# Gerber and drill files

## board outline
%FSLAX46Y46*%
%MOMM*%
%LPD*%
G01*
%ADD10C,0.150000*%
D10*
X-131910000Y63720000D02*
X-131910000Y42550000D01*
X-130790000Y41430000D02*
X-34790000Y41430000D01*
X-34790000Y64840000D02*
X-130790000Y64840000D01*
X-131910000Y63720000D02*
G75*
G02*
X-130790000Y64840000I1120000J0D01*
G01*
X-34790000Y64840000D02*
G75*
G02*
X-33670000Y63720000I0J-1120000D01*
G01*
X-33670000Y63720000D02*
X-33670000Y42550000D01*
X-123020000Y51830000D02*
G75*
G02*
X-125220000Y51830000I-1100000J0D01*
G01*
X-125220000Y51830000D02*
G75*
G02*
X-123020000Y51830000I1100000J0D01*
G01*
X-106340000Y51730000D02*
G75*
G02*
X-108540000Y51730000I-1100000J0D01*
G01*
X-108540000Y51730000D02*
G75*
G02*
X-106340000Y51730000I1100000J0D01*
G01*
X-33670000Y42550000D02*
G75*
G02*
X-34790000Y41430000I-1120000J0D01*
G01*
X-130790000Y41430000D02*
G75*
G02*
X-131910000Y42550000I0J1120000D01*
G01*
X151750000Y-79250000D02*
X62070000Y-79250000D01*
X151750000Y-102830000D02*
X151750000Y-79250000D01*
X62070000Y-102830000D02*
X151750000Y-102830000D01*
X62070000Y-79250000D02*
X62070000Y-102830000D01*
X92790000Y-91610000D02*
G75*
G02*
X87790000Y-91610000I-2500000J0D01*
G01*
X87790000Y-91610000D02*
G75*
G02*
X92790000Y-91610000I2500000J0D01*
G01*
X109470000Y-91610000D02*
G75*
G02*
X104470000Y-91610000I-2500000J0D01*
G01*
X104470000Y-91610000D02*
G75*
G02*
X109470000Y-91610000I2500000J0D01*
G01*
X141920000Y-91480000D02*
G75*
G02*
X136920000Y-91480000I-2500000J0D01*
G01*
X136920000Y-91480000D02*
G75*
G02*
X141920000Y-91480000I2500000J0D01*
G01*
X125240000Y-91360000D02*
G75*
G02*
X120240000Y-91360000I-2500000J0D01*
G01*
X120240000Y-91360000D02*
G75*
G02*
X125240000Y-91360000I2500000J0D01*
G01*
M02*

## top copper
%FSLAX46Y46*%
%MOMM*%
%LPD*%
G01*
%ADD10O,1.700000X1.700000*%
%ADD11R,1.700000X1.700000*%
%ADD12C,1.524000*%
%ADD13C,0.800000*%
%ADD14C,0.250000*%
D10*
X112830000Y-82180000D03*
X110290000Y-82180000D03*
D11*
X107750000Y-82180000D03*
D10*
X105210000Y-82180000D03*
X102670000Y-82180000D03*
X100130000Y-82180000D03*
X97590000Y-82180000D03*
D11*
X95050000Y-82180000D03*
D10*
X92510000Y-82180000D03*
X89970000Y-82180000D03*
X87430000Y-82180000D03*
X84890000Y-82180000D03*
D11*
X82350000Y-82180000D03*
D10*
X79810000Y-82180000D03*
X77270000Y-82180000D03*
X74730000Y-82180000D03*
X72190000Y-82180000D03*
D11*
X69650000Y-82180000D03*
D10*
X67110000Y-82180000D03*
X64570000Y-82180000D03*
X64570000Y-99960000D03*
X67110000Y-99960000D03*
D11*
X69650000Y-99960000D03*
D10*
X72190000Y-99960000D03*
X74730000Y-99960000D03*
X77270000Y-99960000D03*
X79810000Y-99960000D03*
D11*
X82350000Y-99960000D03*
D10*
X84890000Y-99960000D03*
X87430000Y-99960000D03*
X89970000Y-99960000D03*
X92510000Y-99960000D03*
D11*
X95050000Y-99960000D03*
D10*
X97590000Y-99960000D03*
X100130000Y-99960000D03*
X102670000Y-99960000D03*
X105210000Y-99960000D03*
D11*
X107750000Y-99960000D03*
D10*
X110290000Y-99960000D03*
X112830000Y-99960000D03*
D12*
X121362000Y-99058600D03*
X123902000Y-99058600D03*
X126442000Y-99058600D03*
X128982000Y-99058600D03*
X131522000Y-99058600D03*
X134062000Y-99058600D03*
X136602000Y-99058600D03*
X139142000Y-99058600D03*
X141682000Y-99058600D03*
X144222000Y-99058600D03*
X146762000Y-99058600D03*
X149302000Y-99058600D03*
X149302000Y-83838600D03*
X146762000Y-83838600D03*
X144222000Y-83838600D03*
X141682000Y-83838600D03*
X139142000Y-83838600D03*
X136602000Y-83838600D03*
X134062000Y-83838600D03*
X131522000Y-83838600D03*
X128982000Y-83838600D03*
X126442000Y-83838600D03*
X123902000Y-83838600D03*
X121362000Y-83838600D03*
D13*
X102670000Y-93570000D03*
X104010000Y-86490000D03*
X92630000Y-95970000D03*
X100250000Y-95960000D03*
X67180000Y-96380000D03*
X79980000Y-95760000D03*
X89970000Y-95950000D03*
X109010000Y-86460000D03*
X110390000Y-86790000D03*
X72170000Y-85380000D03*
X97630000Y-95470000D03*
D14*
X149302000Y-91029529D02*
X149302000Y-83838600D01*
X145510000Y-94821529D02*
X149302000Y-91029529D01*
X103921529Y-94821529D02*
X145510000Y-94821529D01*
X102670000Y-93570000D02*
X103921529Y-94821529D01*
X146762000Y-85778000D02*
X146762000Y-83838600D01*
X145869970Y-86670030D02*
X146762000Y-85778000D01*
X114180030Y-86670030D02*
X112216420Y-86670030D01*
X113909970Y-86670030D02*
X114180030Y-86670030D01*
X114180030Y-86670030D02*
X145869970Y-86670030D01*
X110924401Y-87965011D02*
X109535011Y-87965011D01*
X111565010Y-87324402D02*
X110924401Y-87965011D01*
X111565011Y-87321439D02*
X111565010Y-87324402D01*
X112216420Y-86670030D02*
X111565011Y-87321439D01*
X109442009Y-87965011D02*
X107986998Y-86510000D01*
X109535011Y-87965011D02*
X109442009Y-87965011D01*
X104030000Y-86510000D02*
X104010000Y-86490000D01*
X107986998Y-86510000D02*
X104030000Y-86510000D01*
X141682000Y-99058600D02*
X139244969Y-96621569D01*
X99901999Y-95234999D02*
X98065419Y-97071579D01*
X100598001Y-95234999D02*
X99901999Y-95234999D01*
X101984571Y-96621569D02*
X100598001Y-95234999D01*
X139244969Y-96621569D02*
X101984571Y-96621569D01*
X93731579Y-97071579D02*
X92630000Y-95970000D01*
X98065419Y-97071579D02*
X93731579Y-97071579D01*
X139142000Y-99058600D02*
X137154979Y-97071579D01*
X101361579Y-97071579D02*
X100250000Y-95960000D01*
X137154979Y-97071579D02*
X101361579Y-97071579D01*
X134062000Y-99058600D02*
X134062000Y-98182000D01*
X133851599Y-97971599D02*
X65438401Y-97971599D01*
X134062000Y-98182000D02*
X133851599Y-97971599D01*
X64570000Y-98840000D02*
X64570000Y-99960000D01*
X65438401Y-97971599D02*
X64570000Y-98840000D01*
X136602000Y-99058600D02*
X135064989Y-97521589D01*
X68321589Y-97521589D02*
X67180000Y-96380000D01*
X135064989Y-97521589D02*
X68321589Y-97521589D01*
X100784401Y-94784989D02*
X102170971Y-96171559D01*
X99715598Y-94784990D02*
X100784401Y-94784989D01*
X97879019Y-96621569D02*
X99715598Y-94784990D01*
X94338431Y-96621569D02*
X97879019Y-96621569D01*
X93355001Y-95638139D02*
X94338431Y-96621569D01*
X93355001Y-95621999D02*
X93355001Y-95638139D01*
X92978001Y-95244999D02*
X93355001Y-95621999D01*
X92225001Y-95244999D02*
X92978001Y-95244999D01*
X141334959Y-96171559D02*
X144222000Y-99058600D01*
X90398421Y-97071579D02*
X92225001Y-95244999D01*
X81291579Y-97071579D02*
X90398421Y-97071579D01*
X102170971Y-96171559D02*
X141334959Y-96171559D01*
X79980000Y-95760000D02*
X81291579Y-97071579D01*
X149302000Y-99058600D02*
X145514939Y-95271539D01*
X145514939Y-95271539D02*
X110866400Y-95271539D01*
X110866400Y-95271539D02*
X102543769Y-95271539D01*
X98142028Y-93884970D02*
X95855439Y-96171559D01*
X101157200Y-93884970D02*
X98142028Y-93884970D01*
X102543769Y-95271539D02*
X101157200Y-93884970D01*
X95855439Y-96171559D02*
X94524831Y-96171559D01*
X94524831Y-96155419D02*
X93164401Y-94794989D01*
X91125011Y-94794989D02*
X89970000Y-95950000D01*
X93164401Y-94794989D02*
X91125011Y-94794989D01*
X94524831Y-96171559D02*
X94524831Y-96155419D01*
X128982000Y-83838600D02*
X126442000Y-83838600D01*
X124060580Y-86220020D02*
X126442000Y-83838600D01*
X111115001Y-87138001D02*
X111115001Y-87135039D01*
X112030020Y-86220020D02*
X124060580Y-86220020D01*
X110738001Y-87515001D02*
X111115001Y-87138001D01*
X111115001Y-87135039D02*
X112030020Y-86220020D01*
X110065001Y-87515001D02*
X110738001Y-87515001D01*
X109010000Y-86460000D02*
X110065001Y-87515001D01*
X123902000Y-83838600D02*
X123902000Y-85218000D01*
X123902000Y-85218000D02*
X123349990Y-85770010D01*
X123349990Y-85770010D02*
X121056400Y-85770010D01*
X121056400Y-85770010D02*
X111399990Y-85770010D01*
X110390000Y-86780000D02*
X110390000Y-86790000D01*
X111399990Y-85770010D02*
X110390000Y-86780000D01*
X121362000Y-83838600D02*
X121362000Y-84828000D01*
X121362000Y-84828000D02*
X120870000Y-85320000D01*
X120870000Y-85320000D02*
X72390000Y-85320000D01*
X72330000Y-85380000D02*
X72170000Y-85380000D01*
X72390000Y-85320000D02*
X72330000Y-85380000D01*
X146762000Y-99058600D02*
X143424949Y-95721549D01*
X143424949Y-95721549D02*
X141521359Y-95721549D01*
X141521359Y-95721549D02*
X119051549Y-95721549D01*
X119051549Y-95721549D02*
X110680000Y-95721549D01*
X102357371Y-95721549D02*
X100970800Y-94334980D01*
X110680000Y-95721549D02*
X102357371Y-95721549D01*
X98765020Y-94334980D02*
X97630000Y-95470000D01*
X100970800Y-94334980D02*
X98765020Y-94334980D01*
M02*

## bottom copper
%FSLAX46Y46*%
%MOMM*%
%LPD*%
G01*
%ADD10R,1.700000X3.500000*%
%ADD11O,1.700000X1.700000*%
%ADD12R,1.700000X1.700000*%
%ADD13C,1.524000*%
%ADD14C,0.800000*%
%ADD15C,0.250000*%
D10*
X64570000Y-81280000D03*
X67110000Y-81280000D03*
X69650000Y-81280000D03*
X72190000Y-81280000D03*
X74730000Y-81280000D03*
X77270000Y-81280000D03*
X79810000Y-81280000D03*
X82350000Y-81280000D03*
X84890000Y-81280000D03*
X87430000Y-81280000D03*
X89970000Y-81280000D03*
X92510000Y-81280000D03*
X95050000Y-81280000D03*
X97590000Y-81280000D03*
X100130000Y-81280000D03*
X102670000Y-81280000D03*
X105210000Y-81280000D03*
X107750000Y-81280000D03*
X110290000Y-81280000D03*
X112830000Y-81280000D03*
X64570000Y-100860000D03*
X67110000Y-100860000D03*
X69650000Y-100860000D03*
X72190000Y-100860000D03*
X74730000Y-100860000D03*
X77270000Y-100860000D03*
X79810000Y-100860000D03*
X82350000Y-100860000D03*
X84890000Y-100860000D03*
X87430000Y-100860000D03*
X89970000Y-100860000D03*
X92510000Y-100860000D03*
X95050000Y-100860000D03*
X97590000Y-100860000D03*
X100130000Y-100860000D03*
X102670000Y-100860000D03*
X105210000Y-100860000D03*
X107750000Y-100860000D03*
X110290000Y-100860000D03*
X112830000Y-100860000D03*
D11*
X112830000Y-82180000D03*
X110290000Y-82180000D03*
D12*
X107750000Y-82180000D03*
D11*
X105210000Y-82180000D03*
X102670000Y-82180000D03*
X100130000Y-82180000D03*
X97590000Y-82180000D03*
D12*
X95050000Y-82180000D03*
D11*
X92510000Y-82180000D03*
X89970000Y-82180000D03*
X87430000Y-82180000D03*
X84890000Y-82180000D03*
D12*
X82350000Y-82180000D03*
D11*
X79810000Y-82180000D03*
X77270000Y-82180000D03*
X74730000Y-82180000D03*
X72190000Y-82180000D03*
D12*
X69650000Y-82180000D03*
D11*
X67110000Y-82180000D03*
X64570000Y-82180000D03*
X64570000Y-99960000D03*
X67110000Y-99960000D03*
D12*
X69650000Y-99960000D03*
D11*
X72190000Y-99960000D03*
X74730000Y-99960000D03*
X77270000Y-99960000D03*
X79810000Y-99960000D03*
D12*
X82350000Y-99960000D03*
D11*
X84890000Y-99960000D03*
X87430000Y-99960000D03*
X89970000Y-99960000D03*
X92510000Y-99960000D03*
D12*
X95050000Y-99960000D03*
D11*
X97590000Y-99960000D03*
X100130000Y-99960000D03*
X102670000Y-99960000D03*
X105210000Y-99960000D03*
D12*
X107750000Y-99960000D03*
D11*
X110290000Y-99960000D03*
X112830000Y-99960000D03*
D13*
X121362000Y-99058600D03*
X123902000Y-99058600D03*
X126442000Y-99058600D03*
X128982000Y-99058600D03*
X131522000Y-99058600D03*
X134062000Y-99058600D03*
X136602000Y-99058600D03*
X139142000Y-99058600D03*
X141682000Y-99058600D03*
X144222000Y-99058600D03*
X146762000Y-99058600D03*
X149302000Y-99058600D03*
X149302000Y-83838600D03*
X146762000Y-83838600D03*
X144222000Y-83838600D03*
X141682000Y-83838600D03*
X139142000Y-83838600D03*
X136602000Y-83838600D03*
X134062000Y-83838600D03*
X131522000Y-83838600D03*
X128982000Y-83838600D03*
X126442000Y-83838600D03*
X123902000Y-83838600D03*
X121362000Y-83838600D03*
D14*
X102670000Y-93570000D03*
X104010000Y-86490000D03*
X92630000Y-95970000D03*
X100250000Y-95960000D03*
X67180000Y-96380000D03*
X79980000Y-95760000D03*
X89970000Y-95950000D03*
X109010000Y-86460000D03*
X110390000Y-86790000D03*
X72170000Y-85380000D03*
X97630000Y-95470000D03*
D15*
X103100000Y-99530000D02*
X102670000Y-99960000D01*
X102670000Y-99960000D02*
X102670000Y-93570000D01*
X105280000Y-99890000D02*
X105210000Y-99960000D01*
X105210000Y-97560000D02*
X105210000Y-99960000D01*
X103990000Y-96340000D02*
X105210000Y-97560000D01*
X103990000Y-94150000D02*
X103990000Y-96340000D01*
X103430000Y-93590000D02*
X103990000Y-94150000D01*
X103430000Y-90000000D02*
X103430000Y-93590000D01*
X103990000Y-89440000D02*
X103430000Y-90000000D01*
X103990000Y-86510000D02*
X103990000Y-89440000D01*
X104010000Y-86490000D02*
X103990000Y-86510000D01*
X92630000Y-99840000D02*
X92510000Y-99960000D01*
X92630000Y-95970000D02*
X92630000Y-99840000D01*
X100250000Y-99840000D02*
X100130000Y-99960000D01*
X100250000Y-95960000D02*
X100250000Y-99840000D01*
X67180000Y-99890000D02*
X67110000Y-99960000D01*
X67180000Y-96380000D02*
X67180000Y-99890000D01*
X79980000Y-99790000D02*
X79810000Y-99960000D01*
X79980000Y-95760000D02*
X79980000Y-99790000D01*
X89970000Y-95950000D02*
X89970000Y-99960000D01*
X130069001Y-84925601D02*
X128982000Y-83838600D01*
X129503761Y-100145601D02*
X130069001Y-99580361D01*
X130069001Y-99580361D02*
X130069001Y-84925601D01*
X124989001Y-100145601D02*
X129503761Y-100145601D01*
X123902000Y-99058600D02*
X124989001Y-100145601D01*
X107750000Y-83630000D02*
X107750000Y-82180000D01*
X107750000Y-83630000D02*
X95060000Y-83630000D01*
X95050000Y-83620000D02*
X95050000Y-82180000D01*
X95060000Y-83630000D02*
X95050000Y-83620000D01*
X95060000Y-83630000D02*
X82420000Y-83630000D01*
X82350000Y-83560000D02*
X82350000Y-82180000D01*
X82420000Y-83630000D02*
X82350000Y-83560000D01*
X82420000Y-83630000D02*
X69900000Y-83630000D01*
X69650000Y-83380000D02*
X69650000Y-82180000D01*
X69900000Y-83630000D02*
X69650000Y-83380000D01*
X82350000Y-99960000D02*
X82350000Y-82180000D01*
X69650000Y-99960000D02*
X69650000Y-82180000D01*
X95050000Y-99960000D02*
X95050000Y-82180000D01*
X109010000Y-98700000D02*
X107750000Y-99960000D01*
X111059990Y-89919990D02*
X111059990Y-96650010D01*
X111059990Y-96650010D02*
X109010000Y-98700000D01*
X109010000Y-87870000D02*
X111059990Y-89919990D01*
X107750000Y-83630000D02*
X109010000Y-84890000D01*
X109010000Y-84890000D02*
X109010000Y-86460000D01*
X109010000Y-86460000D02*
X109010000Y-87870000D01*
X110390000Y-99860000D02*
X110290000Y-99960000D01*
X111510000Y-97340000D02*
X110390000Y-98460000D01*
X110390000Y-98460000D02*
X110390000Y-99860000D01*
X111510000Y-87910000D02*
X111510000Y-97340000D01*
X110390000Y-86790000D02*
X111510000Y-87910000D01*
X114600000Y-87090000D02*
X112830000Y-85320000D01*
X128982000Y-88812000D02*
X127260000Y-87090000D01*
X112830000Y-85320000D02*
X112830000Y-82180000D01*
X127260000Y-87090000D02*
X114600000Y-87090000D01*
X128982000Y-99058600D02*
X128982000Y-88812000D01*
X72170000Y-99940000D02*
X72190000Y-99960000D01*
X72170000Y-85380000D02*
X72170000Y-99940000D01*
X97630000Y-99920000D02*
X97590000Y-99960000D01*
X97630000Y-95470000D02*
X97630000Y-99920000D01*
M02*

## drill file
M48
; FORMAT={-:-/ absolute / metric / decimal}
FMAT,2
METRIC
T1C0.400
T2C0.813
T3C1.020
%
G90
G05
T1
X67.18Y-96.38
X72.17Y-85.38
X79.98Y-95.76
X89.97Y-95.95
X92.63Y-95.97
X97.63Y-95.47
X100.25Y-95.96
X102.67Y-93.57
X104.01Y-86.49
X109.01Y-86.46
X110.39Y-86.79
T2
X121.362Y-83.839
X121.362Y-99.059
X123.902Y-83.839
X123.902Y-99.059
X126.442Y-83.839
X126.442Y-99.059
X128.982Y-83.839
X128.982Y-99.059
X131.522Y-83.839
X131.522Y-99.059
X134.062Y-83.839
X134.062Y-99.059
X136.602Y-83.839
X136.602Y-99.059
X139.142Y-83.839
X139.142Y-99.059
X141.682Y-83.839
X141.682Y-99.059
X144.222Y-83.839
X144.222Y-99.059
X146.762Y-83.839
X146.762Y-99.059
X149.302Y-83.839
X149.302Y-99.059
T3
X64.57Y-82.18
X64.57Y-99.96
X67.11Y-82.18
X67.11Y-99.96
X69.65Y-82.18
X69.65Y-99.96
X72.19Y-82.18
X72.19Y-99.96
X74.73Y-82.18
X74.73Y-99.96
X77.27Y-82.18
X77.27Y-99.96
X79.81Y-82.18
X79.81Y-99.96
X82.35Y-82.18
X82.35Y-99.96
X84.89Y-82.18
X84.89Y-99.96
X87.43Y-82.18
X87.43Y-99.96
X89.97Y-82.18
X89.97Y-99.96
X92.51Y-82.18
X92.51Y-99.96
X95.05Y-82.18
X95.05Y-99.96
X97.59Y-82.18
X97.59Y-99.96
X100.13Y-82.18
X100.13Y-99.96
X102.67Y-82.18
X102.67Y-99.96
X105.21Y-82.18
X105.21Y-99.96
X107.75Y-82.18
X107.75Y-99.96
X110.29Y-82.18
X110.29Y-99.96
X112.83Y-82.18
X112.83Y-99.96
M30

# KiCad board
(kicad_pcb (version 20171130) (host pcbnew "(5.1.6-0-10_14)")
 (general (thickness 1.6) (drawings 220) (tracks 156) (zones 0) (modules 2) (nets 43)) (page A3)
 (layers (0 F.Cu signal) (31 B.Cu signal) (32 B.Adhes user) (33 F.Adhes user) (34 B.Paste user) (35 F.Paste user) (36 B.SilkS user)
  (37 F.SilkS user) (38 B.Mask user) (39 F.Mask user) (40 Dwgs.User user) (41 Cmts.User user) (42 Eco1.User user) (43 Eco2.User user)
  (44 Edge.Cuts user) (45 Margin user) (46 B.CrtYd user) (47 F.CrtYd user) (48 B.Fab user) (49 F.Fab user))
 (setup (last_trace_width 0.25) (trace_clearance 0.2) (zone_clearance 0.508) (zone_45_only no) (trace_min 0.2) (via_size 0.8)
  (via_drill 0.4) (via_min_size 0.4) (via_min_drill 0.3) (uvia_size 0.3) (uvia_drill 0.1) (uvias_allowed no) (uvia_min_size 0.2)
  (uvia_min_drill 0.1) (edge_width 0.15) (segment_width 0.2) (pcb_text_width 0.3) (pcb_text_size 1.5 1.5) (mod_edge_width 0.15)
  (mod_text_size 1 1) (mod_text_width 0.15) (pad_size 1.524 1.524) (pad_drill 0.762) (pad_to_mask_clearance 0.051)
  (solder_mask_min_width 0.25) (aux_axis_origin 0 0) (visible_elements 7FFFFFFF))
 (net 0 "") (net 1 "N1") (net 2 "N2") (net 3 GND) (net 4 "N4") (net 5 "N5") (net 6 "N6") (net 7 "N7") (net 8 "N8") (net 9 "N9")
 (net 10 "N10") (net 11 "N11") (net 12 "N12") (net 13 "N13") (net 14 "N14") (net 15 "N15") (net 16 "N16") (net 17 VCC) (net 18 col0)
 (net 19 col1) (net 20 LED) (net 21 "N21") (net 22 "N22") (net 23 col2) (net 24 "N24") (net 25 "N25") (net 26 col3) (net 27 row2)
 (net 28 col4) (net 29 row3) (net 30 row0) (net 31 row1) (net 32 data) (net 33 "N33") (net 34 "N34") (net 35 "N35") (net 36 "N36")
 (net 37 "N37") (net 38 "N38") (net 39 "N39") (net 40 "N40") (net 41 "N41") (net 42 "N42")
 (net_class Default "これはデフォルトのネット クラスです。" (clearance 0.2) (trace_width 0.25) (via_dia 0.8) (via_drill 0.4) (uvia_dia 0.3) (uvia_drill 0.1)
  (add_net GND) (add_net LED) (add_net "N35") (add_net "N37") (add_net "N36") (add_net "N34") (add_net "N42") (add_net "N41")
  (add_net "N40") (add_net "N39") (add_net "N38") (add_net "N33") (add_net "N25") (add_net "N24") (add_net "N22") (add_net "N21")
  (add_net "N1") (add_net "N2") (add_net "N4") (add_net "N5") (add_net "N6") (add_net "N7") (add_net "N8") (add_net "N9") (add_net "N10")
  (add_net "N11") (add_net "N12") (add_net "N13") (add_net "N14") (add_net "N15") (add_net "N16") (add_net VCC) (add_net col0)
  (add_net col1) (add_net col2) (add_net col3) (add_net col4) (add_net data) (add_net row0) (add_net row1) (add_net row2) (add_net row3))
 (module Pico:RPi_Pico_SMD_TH (layer B.Cu) (at 88.7 91.07 90)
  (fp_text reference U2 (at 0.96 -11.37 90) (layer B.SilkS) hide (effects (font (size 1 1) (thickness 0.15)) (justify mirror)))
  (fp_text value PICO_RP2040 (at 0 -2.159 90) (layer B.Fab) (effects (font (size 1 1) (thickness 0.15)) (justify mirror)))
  (pad 21 smd rect (at 8.89 -24.13 90) (size 3.5 1.7) (drill (offset 0.9 0)) (layers B.Cu B.Mask) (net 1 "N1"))
  (pad 22 smd rect (at 8.89 -21.59 90) (size 3.5 1.7) (drill (offset 0.9 0)) (layers B.Cu B.Mask) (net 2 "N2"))
  (pad 23 smd rect (at 8.89 -19.05 90) (size 3.5 1.7) (drill (offset 0.9 0)) (layers B.Cu B.Mask) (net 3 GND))
  (pad 24 smd rect (at 8.89 -16.51 90) (size 3.5 1.7) (drill (offset 0.9 0)) (layers B.Cu B.Mask) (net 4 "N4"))
  (pad 25 smd rect (at 8.89 -13.97 90) (size 3.5 1.7) (drill (offset 0.9 0)) (layers B.Cu B.Mask) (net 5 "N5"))
  (pad 26 smd rect (at 8.89 -11.43 90) (size 3.5 1.7) (drill (offset 0.9 0)) (layers B.Cu B.Mask) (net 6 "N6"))
  (pad 27 smd rect (at 8.89 -8.89 90) (size 3.5 1.7) (drill (offset 0.9 0)) (layers B.Cu B.Mask) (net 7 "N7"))
  (pad 28 smd rect (at 8.89 -6.35 90) (size 3.5 1.7) (drill (offset 0.9 0)) (layers B.Cu B.Mask) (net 3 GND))
  (pad 29 smd rect (at 8.89 -3.81 90) (size 3.5 1.7) (drill (offset 0.9 0)) (layers B.Cu B.Mask) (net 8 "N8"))
  (pad 30 smd rect (at 8.89 -1.27 90) (size 3.5 1.7) (drill (offset 0.9 0)) (layers B.Cu B.Mask) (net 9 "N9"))
  (pad 31 smd rect (at 8.89 1.27 90) (size 3.5 1.7) (drill (offset 0.9 0)) (layers B.Cu B.Mask) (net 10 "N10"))
  (pad 32 smd rect (at 8.89 3.81 90) (size 3.5 1.7) (drill (offset 0.9 0)) (layers B.Cu B.Mask) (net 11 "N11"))
  (pad 33 smd rect (at 8.89 6.35 90) (size 3.5 1.7) (drill (offset 0.9 0)) (layers B.Cu B.Mask) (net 3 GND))
  (pad 34 smd rect (at 8.89 8.89 90) (size 3.5 1.7) (drill (offset 0.9 0)) (layers B.Cu B.Mask) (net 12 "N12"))
  (pad 35 smd rect (at 8.89 11.43 90) (size 3.5 1.7) (drill (offset 0.9 0)) (layers B.Cu B.Mask) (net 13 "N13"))
  (pad 36 smd rect (at 8.89 13.97 90) (size 3.5 1.7) (drill (offset 0.9 0)) (layers B.Cu B.Mask) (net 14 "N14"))
  (pad 37 smd rect (at 8.89 16.51 90) (size 3.5 1.7) (drill (offset 0.9 0)) (layers B.Cu B.Mask) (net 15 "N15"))
  (pad 38 smd rect (at 8.89 19.05 90) (size 3.5 1.7) (drill (offset 0.9 0)) (layers B.Cu B.Mask) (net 3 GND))
  (pad 39 smd rect (at 8.89 21.59 90) (size 3.5 1.7) (drill (offset 0.9 0)) (layers B.Cu B.Mask) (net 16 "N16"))
  (pad 40 smd rect (at 8.89 24.13 90) (size 3.5 1.7) (drill (offset 0.9 0)) (layers B.Cu B.Mask) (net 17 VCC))
  (pad 20 smd rect (at -8.89 -24.13 90) (size 3.5 1.7) (drill (offset -0.9 0)) (layers B.Cu B.Mask) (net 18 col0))
  (pad 19 smd rect (at -8.89 -21.59 90) (size 3.5 1.7) (drill (offset -0.9 0)) (layers B.Cu B.Mask) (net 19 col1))
  (pad 18 smd rect (at -8.89 -19.05 90) (size 3.5 1.7) (drill (offset -0.9 0)) (layers B.Cu B.Mask) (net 3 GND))
  (pad 17 smd rect (at -8.89 -16.51 90) (size 3.5 1.7) (drill (offset -0.9 0)) (layers B.Cu B.Mask) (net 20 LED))
  (pad 16 smd rect (at -8.89 -13.97 90) (size 3.5 1.7) (drill (offset -0.9 0)) (layers B.Cu B.Mask) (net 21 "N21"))
  (pad 15 smd rect (at -8.89 -11.43 90) (size 3.5 1.7) (drill (offset -0.9 0)) (layers B.Cu B.Mask) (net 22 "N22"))
  (pad 14 smd rect (at -8.89 -8.89 90) (size 3.5 1.7) (drill (offset -0.9 0)) (layers B.Cu B.Mask) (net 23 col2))
  (pad 13 smd rect (at -8.89 -6.35 90) (size 3.5 1.7) (drill (offset -0.9 0)) (layers B.Cu B.Mask) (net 3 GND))
  (pad 12 smd rect (at -8.89 -3.81 90) (size 3.5 1.7) (drill (offset -0.9 0)) (layers B.Cu B.Mask) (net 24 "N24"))
  (pad 11 smd rect (at -8.89 -1.27 90) (size 3.5 1.7) (drill (offset -0.9 0)) (layers B.Cu B.Mask) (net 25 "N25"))
  (pad 10 smd rect (at -8.89 1.27 90) (size 3.5 1.7) (drill (offset -0.9 0)) (layers B.Cu B.Mask) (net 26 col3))
  (pad 9 smd rect (at -8.89 3.81 90) (size 3.5 1.7) (drill (offset -0.9 0)) (layers B.Cu B.Mask) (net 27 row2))
  (pad 8 smd rect (at -8.89 6.35 90) (size 3.5 1.7) (drill (offset -0.9 0)) (layers B.Cu B.Mask) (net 3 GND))
  (pad 7 smd rect (at -8.89 8.89 90) (size 3.5 1.7) (drill (offset -0.9 0)) (layers B.Cu B.Mask) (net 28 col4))
  (pad 6 smd rect (at -8.89 11.43 90) (size 3.5 1.7) (drill (offset -0.9 0)) (layers B.Cu B.Mask) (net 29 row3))
  (pad 5 smd rect (at -8.89 13.97 90) (size 3.5 1.7) (drill (offset -0.9 0)) (layers B.Cu B.Mask) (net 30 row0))
  (pad 4 smd rect (at -8.89 16.51 90) (size 3.5 1.7) (drill (offset -0.9 0)) (layers B.Cu B.Mask) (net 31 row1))
  (pad 3 smd rect (at -8.89 19.05 90) (size 3.5 1.7) (drill (offset -0.9 0)) (layers B.Cu B.Mask) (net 3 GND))
  (pad 2 smd rect (at -8.89 21.59 90) (size 3.5 1.7) (drill (offset -0.9 0)) (layers B.Cu B.Mask) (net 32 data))
  (pad 1 smd rect (at -8.89 24.13 90) (size 3.5 1.7) (drill (offset -0.9 0)) (layers B.Cu B.Mask) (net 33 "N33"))
  (pad 40 thru_hole oval (at 8.89 24.13 90) (size 1.7 1.7) (drill 1.02) (layers *.Cu *.Mask) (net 17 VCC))
  (pad 39 thru_hole oval (at 8.89 21.59 90) (size 1.7 1.7) (drill 1.02) (layers *.Cu *.Mask) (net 16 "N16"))
  (pad 38 thru_hole rect (at 8.89 19.05 90) (size 1.7 1.7) (drill 1.02) (layers *.Cu *.Mask) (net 3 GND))
  (pad 37 thru_hole oval (at 8.89 16.51 90) (size 1.7 1.7) (drill 1.02) (layers *.Cu *.Mask) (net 15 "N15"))
  (pad 36 thru_hole oval (at 8.89 13.97 90) (size 1.7 1.7) (drill 1.02) (layers *.Cu *.Mask) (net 14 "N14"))
  (pad 35 thru_hole oval (at 8.89 11.43 90) (size 1.7 1.7) (drill 1.02) (layers *.Cu *.Mask) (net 13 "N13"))
  (pad 34 thru_hole oval (at 8.89 8.89 90) (size 1.7 1.7) (drill 1.02) (layers *.Cu *.Mask) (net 12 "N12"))
  (pad 33 thru_hole rect (at 8.89 6.35 90) (size 1.7 1.7) (drill 1.02) (layers *.Cu *.Mask) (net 3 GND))
  (pad 32 thru_hole oval (at 8.89 3.81 90) (size 1.7 1.7) (drill 1.02) (layers *.Cu *.Mask) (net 11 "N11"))
  (pad 31 thru_hole oval (at 8.89 1.27 90) (size 1.7 1.7) (drill 1.02) (layers *.Cu *.Mask) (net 10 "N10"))
  (pad 30 thru_hole oval (at 8.89 -1.27 90) (size 1.7 1.7) (drill 1.02) (layers *.Cu *.Mask) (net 9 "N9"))
  (pad 29 thru_hole oval (at 8.89 -3.81 90) (size 1.7 1.7) (drill 1.02) (layers *.Cu *.Mask) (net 8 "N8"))
  (pad 28 thru_hole rect (at 8.89 -6.35 90) (size 1.7 1.7) (drill 1.02) (layers *.Cu *.Mask) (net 3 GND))
  (pad 27 thru_hole oval (at 8.89 -8.89 90) (size 1.7 1.7) (drill 1.02) (layers *.Cu *.Mask) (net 7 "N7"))
  (pad 26 thru_hole oval (at 8.89 -11.43 90) (size 1.7 1.7) (drill 1.02) (layers *.Cu *.Mask) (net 6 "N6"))
  (pad 25 thru_hole oval (at 8.89 -13.97 90) (size 1.7 1.7) (drill 1.02) (layers *.Cu *.Mask) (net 5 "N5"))
  (pad 24 thru_hole oval (at 8.89 -16.51 90) (size 1.7 1.7) (drill 1.02) (layers *.Cu *.Mask) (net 4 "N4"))
  (pad 23 thru_hole rect (at 8.89 -19.05 90) (size 1.7 1.7) (drill 1.02) (layers *.Cu *.Mask) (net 3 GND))
  (pad 22 thru_hole oval (at 8.89 -21.59 90) (size 1.7 1.7) (drill 1.02) (layers *.Cu *.Mask) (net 2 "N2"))
  (pad 21 thru_hole oval (at 8.89 -24.13 90) (size 1.7 1.7) (drill 1.02) (layers *.Cu *.Mask) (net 1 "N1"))
  (pad 20 thru_hole oval (at -8.89 -24.13 90) (size 1.7 1.7) (drill 1.02) (layers *.Cu *.Mask) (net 18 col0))
  (pad 19 thru_hole oval (at -8.89 -21.59 90) (size 1.7 1.7) (drill 1.02) (layers *.Cu *.Mask) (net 19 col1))
  (pad 18 thru_hole rect (at -8.89 -19.05 90) (size 1.7 1.7) (drill 1.02) (layers *.Cu *.Mask) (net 3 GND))
  (pad 17 thru_hole oval (at -8.89 -16.51 90) (size 1.7 1.7) (drill 1.02) (layers *.Cu *.Mask) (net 20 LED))
  (pad 16 thru_hole oval (at -8.89 -13.97 90) (size 1.7 1.7) (drill 1.02) (layers *.Cu *.Mask) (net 21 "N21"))
  (pad 15 thru_hole oval (at -8.89 -11.43 90) (size 1.7 1.7) (drill 1.02) (layers *.Cu *.Mask) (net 22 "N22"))
  (pad 14 thru_hole oval (at -8.89 -8.89 90) (size 1.7 1.7) (drill 1.02) (layers *.Cu *.Mask) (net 23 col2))
  (pad 13 thru_hole rect (at -8.89 -6.35 90) (size 1.7 1.7) (drill 1.02) (layers *.Cu *.Mask) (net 3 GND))
  (pad 12 thru_hole oval (at -8.89 -3.81 90) (size 1.7 1.7) (drill 1.02) (layers *.Cu *.Mask) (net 24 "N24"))
  (pad 11 thru_hole oval (at -8.89 -1.27 90) (size 1.7 1.7) (drill 1.02) (layers *.Cu *.Mask) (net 25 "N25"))
  (pad 10 thru_hole oval (at -8.89 1.27 90) (size 1.7 1.7) (drill 1.02) (layers *.Cu *.Mask) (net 26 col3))
  (pad 9 thru_hole oval (at -8.89 3.81 90) (size 1.7 1.7) (drill 1.02) (layers *.Cu *.Mask) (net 27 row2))
  (pad 8 thru_hole rect (at -8.89 6.35 90) (size 1.7 1.7) (drill 1.02) (layers *.Cu *.Mask) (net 3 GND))
  (pad 7 thru_hole oval (at -8.89 8.89 90) (size 1.7 1.7) (drill 1.02) (layers *.Cu *.Mask) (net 28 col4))
  (pad 6 thru_hole oval (at -8.89 11.43 90) (size 1.7 1.7) (drill 1.02) (layers *.Cu *.Mask) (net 29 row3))
  (pad 5 thru_hole oval (at -8.89 13.97 90) (size 1.7 1.7) (drill 1.02) (layers *.Cu *.Mask) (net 30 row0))
  (pad 4 thru_hole oval (at -8.89 16.51 90) (size 1.7 1.7) (drill 1.02) (layers *.Cu *.Mask) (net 31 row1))
  (pad 3 thru_hole rect (at -8.89 19.05 90) (size 1.7 1.7) (drill 1.02) (layers *.Cu *.Mask) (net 3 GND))
  (pad 2 thru_hole oval (at -8.89 21.59 90) (size 1.7 1.7) (drill 1.02) (layers *.Cu *.Mask) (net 32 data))
  (pad 1 thru_hole oval (at -8.89 24.13 90) (size 1.7 1.7) (drill 1.02) (layers *.Cu *.Mask) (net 33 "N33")))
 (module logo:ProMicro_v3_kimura (layer F.Cu) (at 135.84 91.45 90)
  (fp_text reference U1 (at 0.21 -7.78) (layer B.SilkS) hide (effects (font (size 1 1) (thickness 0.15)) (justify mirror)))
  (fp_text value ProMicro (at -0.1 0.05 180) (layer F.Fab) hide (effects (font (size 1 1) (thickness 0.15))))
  (pad 24 thru_hole circle (at -7.6086 -14.478 90) (size 1.524 1.524) (drill 0.8128) (layers *.Cu F.SilkS B.Mask) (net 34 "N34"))
  (pad 23 thru_hole circle (at -7.6086 -11.938 90) (size 1.524 1.524) (drill 0.8128) (layers *.Cu F.SilkS B.Mask) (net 3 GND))
  (pad 22 thru_hole circle (at -7.6086 -9.398 90) (size 1.524 1.524) (drill 0.8128) (layers *.Cu F.SilkS B.Mask) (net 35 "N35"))
  (pad 21 thru_hole circle (at -7.6086 -6.858 90) (size 1.524 1.524) (drill 0.8128) (layers *.Cu F.SilkS B.Mask) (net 17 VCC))
  (pad 20 thru_hole circle (at -7.6086 -4.318 90) (size 1.524 1.524) (drill 0.8128) (layers *.Cu F.SilkS B.Mask) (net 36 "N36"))
  (pad 19 thru_hole circle (at -7.6086 -1.778 90) (size 1.524 1.524) (drill 0.8128) (layers *.Cu F.SilkS B.Mask) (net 18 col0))
  (pad 18 thru_hole circle (at -7.6086 0.762 90) (size 1.524 1.524) (drill 0.8128) (layers *.Cu F.SilkS B.Mask) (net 19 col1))
  (pad 17 thru_hole circle (at -7.6086 3.302 90) (size 1.524 1.524) (drill 0.8128) (layers *.Cu F.SilkS B.Mask) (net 29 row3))
  (pad 16 thru_hole circle (at -7.6086 5.842 90) (size 1.524 1.524) (drill 0.8128) (layers *.Cu F.SilkS B.Mask) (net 27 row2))
  (pad 15 thru_hole circle (at -7.6086 8.382 90) (size 1.524 1.524) (drill 0.8128) (layers *.Cu F.SilkS B.Mask) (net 23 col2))
  (pad 14 thru_hole circle (at -7.6086 10.922 90) (size 1.524 1.524) (drill 0.8128) (layers *.Cu F.SilkS B.Mask) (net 28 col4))
  (pad 13 thru_hole circle (at -7.6086 13.462 90) (size 1.524 1.524) (drill 0.8128) (layers *.Cu F.SilkS B.Mask) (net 26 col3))
  (pad 12 thru_hole circle (at 7.6114 13.462 90) (size 1.524 1.524) (drill 0.8128) (layers *.Cu F.SilkS B.Mask) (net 30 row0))
  (pad 11 thru_hole circle (at 7.6114 10.922 90) (size 1.524 1.524) (drill 0.8128) (layers *.Cu F.SilkS B.Mask) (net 31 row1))
  (pad 10 thru_hole circle (at 7.6114 8.382 90) (size 1.524 1.524) (drill 0.8128) (layers *.Cu F.SilkS B.Mask) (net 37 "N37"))
  (pad 9 thru_hole circle (at 7.6114 5.842 90) (size 1.524 1.524) (drill 0.8128) (layers *.Cu F.SilkS B.Mask) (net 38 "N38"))
  (pad 8 thru_hole circle (at 7.6114 3.302 90) (size 1.524 1.524) (drill 0.8128) (layers *.Cu F.SilkS B.Mask) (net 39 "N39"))
  (pad 7 thru_hole circle (at 7.6114 0.762 90) (size 1.524 1.524) (drill 0.8128) (layers *.Cu F.SilkS B.Mask) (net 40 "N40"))
  (pad 6 thru_hole circle (at 7.6114 -1.778 90) (size 1.524 1.524) (drill 0.8128) (layers *.Cu F.SilkS B.Mask) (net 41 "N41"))
  (pad 5 thru_hole circle (at 7.6114 -4.318 90) (size 1.524 1.524) (drill 0.8128) (layers *.Cu F.SilkS B.Mask) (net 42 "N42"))
  (pad 4 thru_hole circle (at 7.6114 -6.858 90) (size 1.524 1.524) (drill 0.8128) (layers *.Cu F.SilkS B.Mask) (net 3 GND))
  (pad 3 thru_hole circle (at 7.6114 -9.398 90) (size 1.524 1.524) (drill 0.8128) (layers *.Cu F.SilkS B.Mask) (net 3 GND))
  (pad 2 thru_hole circle (at 7.6114 -11.938 90) (size 1.524 1.524) (drill 0.8128) (layers *.Cu F.SilkS B.Mask) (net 32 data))
  (pad 1 thru_hole circle (at 7.6114 -14.478 90) (size 1.524 1.524) (drill 0.8128) (layers *.Cu F.SilkS B.Mask) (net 20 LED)))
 (gr_line (start -131.91 -63.72) (end -131.91 -42.55) (layer Edge.Cuts) (width 0.15))
 (gr_line (start -130.79 -41.43) (end -34.79 -41.43) (layer Edge.Cuts) (width 0.15))
 (gr_line (start -34.79 -64.84) (end -130.79 -64.84) (layer Edge.Cuts) (width 0.15))
 (gr_arc (start -130.79 -63.72) (end -130.79 -64.84) (angle -90) (layer Edge.Cuts) (width 0.15))
 (gr_arc (start -34.79 -63.72) (end -33.67 -63.72) (angle -90) (layer Edge.Cuts) (width 0.15))
 (gr_line (start -33.67 -63.72) (end -33.67 -42.55) (layer Edge.Cuts) (width 0.15))
 (gr_circle (center -124.12 -51.83) (end -123.02 -51.83) (layer Edge.Cuts) (width 0.15))
 (gr_circle (center -107.44 -51.73) (end -106.34 -51.73) (layer Edge.Cuts) (width 0.15))
 (gr_arc (start -34.79 -42.55) (end -34.79 -41.43) (angle -90) (layer Edge.Cuts) (width 0.15))
 (gr_arc (start -130.79 -42.55) (end -131.91 -42.55) (angle -90) (layer Edge.Cuts) (width 0.15))
 (gr_line (start 151.75 79.25) (end 62.07 79.25) (layer Edge.Cuts) (width 0.15))
 (gr_line (start 151.75 102.83) (end 151.75 79.25) (layer Edge.Cuts) (width 0.15))
 (gr_line (start 62.07 102.83) (end 151.75 102.83) (layer Edge.Cuts) (width 0.15))
 (gr_line (start 62.07 79.25) (end 62.07 102.83) (layer Edge.Cuts) (width 0.15))
 (gr_circle (center 90.29 91.61) (end 92.79 91.61) (layer Edge.Cuts) (width 0.15))
 (gr_circle (center 106.97 91.61) (end 109.47 91.61) (layer Edge.Cuts) (width 0.15))
 (gr_circle (center 139.42 91.48) (end 141.92 91.48) (layer Edge.Cuts) (width 0.15))
 (gr_circle (center 122.74 91.36) (end 125.24 91.36) (layer Edge.Cuts) (width 0.15))
 (segment (start 103.1 99.53) (end 102.67 99.96) (width 0.25) (layer B.Cu) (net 30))
 (via (at 102.67 93.57) (size 0.8) (drill 0.4) (layers F.Cu B.Cu) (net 30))
 (segment (start 102.67 99.96) (end 102.67 93.57) (width 0.25) (layer B.Cu) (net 30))
 (segment (start 149.302 91.029529) (end 149.302 83.8386) (width 0.25) (layer F.Cu) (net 30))
 (segment (start 145.51 94.821529) (end 149.302 91.029529) (width 0.25) (layer F.Cu) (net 30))
 (segment (start 103.921529 94.821529) (end 145.51 94.821529) (width 0.25) (layer F.Cu) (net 30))
 (segment (start 102.67 93.57) (end 103.921529 94.821529) (width 0.25) (layer F.Cu) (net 30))
 (segment (start 105.28 99.89) (end 105.21 99.96) (width 0.25) (layer B.Cu) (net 31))
 (segment (start 146.762 85.778) (end 146.762 83.8386) (width 0.25) (layer F.Cu) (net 31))
 (segment (start 145.86997 86.67003) (end 146.762 85.778) (width 0.25) (layer F.Cu) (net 31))
 (segment (start 114.18003 86.67003) (end 112.21642 86.67003) (width 0.25) (layer F.Cu) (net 31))
 (segment (start 113.90997 86.67003) (end 114.18003 86.67003) (width 0.25) (layer F.Cu) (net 31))
 (segment (start 114.18003 86.67003) (end 145.86997 86.67003) (width 0.25) (layer F.Cu) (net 31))
 (segment (start 110.924401 87.965011) (end 109.535011 87.965011) (width 0.25) (layer F.Cu) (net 31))
 (segment (start 111.56501 87.324402) (end 110.924401 87.965011) (width 0.25) (layer F.Cu) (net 31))
 (segment (start 111.565011 87.321439) (end 111.56501 87.324402) (width 0.25) (layer F.Cu) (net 31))
 (segment (start 112.21642 86.67003) (end 111.565011 87.321439) (width 0.25) (layer F.Cu) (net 31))
 (segment (start 109.442009 87.965011) (end 107.986998 86.51) (width 0.25) (layer F.Cu) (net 31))
 (segment (start 109.535011 87.965011) (end 109.442009 87.965011) (width 0.25) (layer F.Cu) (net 31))
 (via (at 104.01 86.49) (size 0.8) (drill 0.4) (layers F.Cu B.Cu) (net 31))
 (segment (start 104.03 86.51) (end 104.01 86.49) (width 0.25) (layer F.Cu) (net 31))
 (segment (start 107.986998 86.51) (end 104.03 86.51) (width 0.25) (layer F.Cu) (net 31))
 (segment (start 105.21 97.56) (end 105.21 99.96) (width 0.25) (layer B.Cu) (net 31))
 (segment (start 103.99 96.34) (end 105.21 97.56) (width 0.25) (layer B.Cu) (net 31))
 (segment (start 103.99 94.15) (end 103.99 96.34) (width 0.25) (layer B.Cu) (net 31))
 (segment (start 103.43 93.59) (end 103.99 94.15) (width 0.25) (layer B.Cu) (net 31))
 (segment (start 103.43 90) (end 103.43 93.59) (width 0.25) (layer B.Cu) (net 31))
 (segment (start 103.99 89.44) (end 103.43 90) (width 0.25) (layer B.Cu) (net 31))
 (segment (start 103.99 86.51) (end 103.99 89.44) (width 0.25) (layer B.Cu) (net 31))
 (segment (start 104.01 86.49) (end 103.99 86.51) (width 0.25) (layer B.Cu) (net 31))
 (segment (start 141.682 99.0586) (end 139.244969 96.621569) (width 0.25) (layer F.Cu) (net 27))
 (segment (start 99.901999 95.234999) (end 98.065419 97.071579) (width 0.25) (layer F.Cu) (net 27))
 (segment (start 100.598001 95.234999) (end 99.901999 95.234999) (width 0.25) (layer F.Cu) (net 27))
 (segment (start 101.984571 96.621569) (end 100.598001 95.234999) (width 0.25) (layer F.Cu) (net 27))
 (segment (start 139.244969 96.621569) (end 101.984571 96.621569) (width 0.25) (layer F.Cu) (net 27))
 (segment (start 93.731579 97.071579) (end 92.63 95.97) (width 0.25) (layer F.Cu) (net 27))
 (via (at 92.63 95.97) (size 0.8) (drill 0.4) (layers F.Cu B.Cu) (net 27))
 (segment (start 98.065419 97.071579) (end 93.731579 97.071579) (width 0.25) (layer F.Cu) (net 27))
 (segment (start 92.63 99.84) (end 92.51 99.96) (width 0.25) (layer B.Cu) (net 27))
 (segment (start 92.63 95.97) (end 92.63 99.84) (width 0.25) (layer B.Cu) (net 27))
 (segment (start 139.142 99.0586) (end 137.154979 97.071579) (width 0.25) (layer F.Cu) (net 29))
 (via (at 100.25 95.96) (size 0.8) (drill 0.4) (layers F.Cu B.Cu) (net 29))
 (segment (start 101.361579 97.071579) (end 100.25 95.96) (width 0.25) (layer F.Cu) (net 29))
 (segment (start 137.154979 97.071579) (end 101.361579 97.071579) (width 0.25) (layer F.Cu) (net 29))
 (segment (start 100.25 99.84) (end 100.13 99.96) (width 0.25) (layer B.Cu) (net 29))
 (segment (start 100.25 95.96) (end 100.25 99.84) (width 0.25) (layer B.Cu) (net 29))
 (segment (start 134.062 99.0586) (end 134.062 98.182) (width 0.25) (layer F.Cu) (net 18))
 (segment (start 133.851599 97.971599) (end 65.438401 97.971599) (width 0.25) (layer F.Cu) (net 18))
 (segment (start 134.062 98.182) (end 133.851599 97.971599) (width 0.25) (layer F.Cu) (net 18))
 (segment (start 64.57 98.84) (end 64.57 99.96) (width 0.25) (layer F.Cu) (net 18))
 (segment (start 65.438401 97.971599) (end 64.57 98.84) (width 0.25) (layer F.Cu) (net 18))
 (segment (start 136.602 99.0586) (end 135.064989 97.521589) (width 0.25) (layer F.Cu) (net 19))
 (via (at 67.18 96.38) (size 0.8) (drill 0.4) (layers F.Cu B.Cu) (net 19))
 (segment (start 68.321589 97.521589) (end 67.18 96.38) (width 0.25) (layer F.Cu) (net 19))
 (segment (start 135.064989 97.521589) (end 68.321589 97.521589) (width 0.25) (layer F.Cu) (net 19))
 (segment (start 67.18 99.89) (end 67.11 99.96) (width 0.25) (layer B.Cu) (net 19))
 (segment (start 67.18 96.38) (end 67.18 99.89) (width 0.25) (layer B.Cu) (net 19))
 (via (at 79.98 95.76) (size 0.8) (drill 0.4) (layers F.Cu B.Cu) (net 23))
 (segment (start 79.98 99.79) (end 79.81 99.96) (width 0.25) (layer B.Cu) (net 23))
 (segment (start 79.98 95.76) (end 79.98 99.79) (width 0.25) (layer B.Cu) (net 23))
 (segment (start 100.784401 94.784989) (end 102.170971 96.171559) (width 0.25) (layer F.Cu) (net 23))
 (segment (start 99.715598 94.78499) (end 100.784401 94.784989) (width 0.25) (layer F.Cu) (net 23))
 (segment (start 97.879019 96.621569) (end 99.715598 94.78499) (width 0.25) (layer F.Cu) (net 23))
 (segment (start 94.338431 96.621569) (end 97.879019 96.621569) (width 0.25) (layer F.Cu) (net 23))
 (segment (start 93.355001 95.638139) (end 94.338431 96.621569) (width 0.25) (layer F.Cu) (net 23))
 (segment (start 93.355001 95.621999) (end 93.355001 95.638139) (width 0.25) (layer F.Cu) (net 23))
 (segment (start 92.978001 95.244999) (end 93.355001 95.621999) (width 0.25) (layer F.Cu) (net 23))
 (segment (start 92.225001 95.244999) (end 92.978001 95.244999) (width 0.25) (layer F.Cu) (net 23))
 (segment (start 141.334959 96.171559) (end 144.222 99.0586) (width 0.25) (layer F.Cu) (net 23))
 (segment (start 90.398421 97.071579) (end 92.225001 95.244999) (width 0.25) (layer F.Cu) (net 23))
 (segment (start 81.291579 97.071579) (end 90.398421 97.071579) (width 0.25) (layer F.Cu) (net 23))
 (segment (start 102.170971 96.171559) (end 141.334959 96.171559) (width 0.25) (layer F.Cu) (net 23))
 (segment (start 79.98 95.76) (end 81.291579 97.071579) (width 0.25) (layer F.Cu) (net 23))
 (segment (start 149.302 99.0586) (end 145.514939 95.271539) (width 0.25) (layer F.Cu) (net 26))
 (segment (start 145.514939 95.271539) (end 110.8664 95.271539) (width 0.25) (layer F.Cu) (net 26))
 (segment (start 110.8664 95.271539) (end 102.543769 95.271539) (width 0.25) (layer F.Cu) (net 26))
 (segment (start 98.142028 93.88497) (end 95.855439 96.171559) (width 0.25) (layer F.Cu) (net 26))
 (segment (start 101.1572 93.88497) (end 98.142028 93.88497) (width 0.25) (layer F.Cu) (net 26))
 (segment (start 102.543769 95.271539) (end 101.1572 93.88497) (width 0.25) (layer F.Cu) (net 26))
 (segment (start 95.855439 96.171559) (end 94.524831 96.171559) (width 0.25) (layer F.Cu) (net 26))
 (via (at 89.97 95.95) (size 0.8) (drill 0.4) (layers F.Cu B.Cu) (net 26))
 (segment (start 94.524831 96.155419) (end 93.164401 94.794989) (width 0.25) (layer F.Cu) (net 26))
 (segment (start 91.125011 94.794989) (end 89.97 95.95) (width 0.25) (layer F.Cu) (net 26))
 (segment (start 93.164401 94.794989) (end 91.125011 94.794989) (width 0.25) (layer F.Cu) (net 26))
 (segment (start 94.524831 96.171559) (end 94.524831 96.155419) (width 0.25) (layer F.Cu) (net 26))
 (segment (start 89.97 95.95) (end 89.97 99.96) (width 0.25) (layer B.Cu) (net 26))
 (segment (start 128.982 83.8386) (end 126.442 83.8386) (width 0.25) (layer F.Cu) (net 3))
 (segment (start 130.069001 84.925601) (end 128.982 83.8386) (width 0.25) (layer B.Cu) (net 3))
 (segment (start 129.503761 100.145601) (end 130.069001 99.580361) (width 0.25) (layer B.Cu) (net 3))
 (segment (start 130.069001 99.580361) (end 130.069001 84.925601) (width 0.25) (layer B.Cu) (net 3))
 (segment (start 124.989001 100.145601) (end 129.503761 100.145601) (width 0.25) (layer B.Cu) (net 3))
 (segment (start 123.902 99.0586) (end 124.989001 100.145601) (width 0.25) (layer B.Cu) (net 3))
 (segment (start 107.75 83.63) (end 107.75 82.18) (width 0.25) (layer B.Cu) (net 3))
 (segment (start 107.75 83.63) (end 95.06 83.63) (width 0.25) (layer B.Cu) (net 3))
 (segment (start 95.05 83.62) (end 95.05 82.18) (width 0.25) (layer B.Cu) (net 3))
 (segment (start 95.06 83.63) (end 95.05 83.62) (width 0.25) (layer B.Cu) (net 3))
 (segment (start 95.06 83.63) (end 82.42 83.63) (width 0.25) (layer B.Cu) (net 3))
 (segment (start 82.35 83.56) (end 82.35 82.18) (width 0.25) (layer B.Cu) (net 3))
 (segment (start 82.42 83.63) (end 82.35 83.56) (width 0.25) (layer B.Cu) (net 3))
 (segment (start 82.42 83.63) (end 69.9 83.63) (width 0.25) (layer B.Cu) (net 3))
 (segment (start 69.65 83.38) (end 69.65 82.18) (width 0.25) (layer B.Cu) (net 3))
 (segment (start 69.9 83.63) (end 69.65 83.38) (width 0.25) (layer B.Cu) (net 3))
 (segment (start 82.35 99.96) (end 82.35 82.18) (width 0.25) (layer B.Cu) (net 3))
 (segment (start 69.65 99.96) (end 69.65 82.18) (width 0.25) (layer B.Cu) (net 3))
 (segment (start 95.05 99.96) (end 95.05 82.18) (width 0.25) (layer B.Cu) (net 3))
 (segment (start 109.01 98.7) (end 107.75 99.96) (width 0.25) (layer B.Cu) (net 3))
 (segment (start 111.05999 89.91999) (end 111.05999 96.65001) (width 0.25) (layer B.Cu) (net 3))
 (segment (start 111.05999 96.65001) (end 109.01 98.7) (width 0.25) (layer B.Cu) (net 3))
 (segment (start 109.01 87.87) (end 111.05999 89.91999) (width 0.25) (layer B.Cu) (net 3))
 (segment (start 107.75 83.63) (end 109.01 84.89) (width 0.25) (layer B.Cu) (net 3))
 (via (at 109.01 86.46) (size 0.8) (drill 0.4) (layers F.Cu B.Cu) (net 3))
 (segment (start 109.01 84.89) (end 109.01 86.46) (width 0.25) (layer B.Cu) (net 3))
 (segment (start 109.01 86.46) (end 109.01 87.87) (width 0.25) (layer B.Cu) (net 3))
 (segment (start 124.06058 86.22002) (end 126.442 83.8386) (width 0.25) (layer F.Cu) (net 3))
 (segment (start 111.115001 87.138001) (end 111.115001 87.135039) (width 0.25) (layer F.Cu) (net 3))
 (segment (start 112.03002 86.22002) (end 124.06058 86.22002) (width 0.25) (layer F.Cu) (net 3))
 (segment (start 110.738001 87.515001) (end 111.115001 87.138001) (width 0.25) (layer F.Cu) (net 3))
 (segment (start 111.115001 87.135039) (end 112.03002 86.22002) (width 0.25) (layer F.Cu) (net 3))
 (segment (start 110.065001 87.515001) (end 110.738001 87.515001) (width 0.25) (layer F.Cu) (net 3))
 (segment (start 109.01 86.46) (end 110.065001 87.515001) (width 0.25) (layer F.Cu) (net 3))
 (segment (start 123.902 83.8386) (end 123.902 85.218) (width 0.25) (layer F.Cu) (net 32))
 (segment (start 123.902 85.218) (end 123.34999 85.77001) (width 0.25) (layer F.Cu) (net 32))
 (segment (start 123.34999 85.77001) (end 121.0564 85.77001) (width 0.25) (layer F.Cu) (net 32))
 (segment (start 121.0564 85.77001) (end 111.39999 85.77001) (width 0.25) (layer F.Cu) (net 32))
 (segment (start 110.39 86.78) (end 110.39 86.79) (width 0.25) (layer F.Cu) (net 32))
 (via (at 110.39 86.79) (size 0.8) (drill 0.4) (layers F.Cu B.Cu) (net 32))
 (segment (start 111.39999 85.77001) (end 110.39 86.78) (width 0.25) (layer F.Cu) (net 32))
 (segment (start 110.39 99.86) (end 110.29 99.96) (width 0.25) (layer B.Cu) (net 32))
 (segment (start 111.51 97.34) (end 110.39 98.46) (width 0.25) (layer B.Cu) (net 32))
 (segment (start 110.39 98.46) (end 110.39 99.86) (width 0.25) (layer B.Cu) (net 32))
 (segment (start 111.51 87.91) (end 111.51 97.34) (width 0.25) (layer B.Cu) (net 32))
 (segment (start 110.39 86.79) (end 111.51 87.91) (width 0.25) (layer B.Cu) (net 32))
 (segment (start 114.6 87.09) (end 112.83 85.32) (width 0.25) (layer B.Cu) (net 17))
 (segment (start 128.982 88.812) (end 127.26 87.09) (width 0.25) (layer B.Cu) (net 17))
 (segment (start 112.83 85.32) (end 112.83 82.18) (width 0.25) (layer B.Cu) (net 17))
 (segment (start 127.26 87.09) (end 114.6 87.09) (width 0.25) (layer B.Cu) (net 17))
 (segment (start 128.982 99.0586) (end 128.982 88.812) (width 0.25) (layer B.Cu) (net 17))
 (segment (start 121.362 83.8386) (end 121.362 84.828) (width 0.25) (layer F.Cu) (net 20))
 (segment (start 121.362 84.828) (end 120.87 85.32) (width 0.25) (layer F.Cu) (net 20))
 (segment (start 120.87 85.32) (end 72.39 85.32) (width 0.25) (layer F.Cu) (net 20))
 (via (at 72.17 85.38) (size 0.8) (drill 0.4) (layers F.Cu B.Cu) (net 20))
 (segment (start 72.33 85.38) (end 72.17 85.38) (width 0.25) (layer F.Cu) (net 20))
 (segment (start 72.39 85.32) (end 72.33 85.38) (width 0.25) (layer F.Cu) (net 20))
 (segment (start 72.17 99.94) (end 72.19 99.96) (width 0.25) (layer B.Cu) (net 20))
 (segment (start 72.17 85.38) (end 72.17 99.94) (width 0.25) (layer B.Cu) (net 20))
 (segment (start 146.762 99.0586) (end 143.424949 95.721549) (width 0.25) (layer F.Cu) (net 28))
 (segment (start 143.424949 95.721549) (end 141.521359 95.721549) (width 0.25) (layer F.Cu) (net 28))
 (segment (start 141.521359 95.721549) (end 119.051549 95.721549) (width 0.25) (layer F.Cu) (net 28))
 (segment (start 119.051549 95.721549) (end 110.68 95.721549) (width 0.25) (layer F.Cu) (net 28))
 (segment (start 102.357371 95.721549) (end 100.9708 94.33498) (width 0.25) (layer F.Cu) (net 28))
 (segment (start 110.68 95.721549) (end 102.357371 95.721549) (width 0.25) (layer F.Cu) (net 28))
 (via (at 97.63 95.47) (size 0.8) (drill 0.4) (layers F.Cu B.Cu) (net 28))
 (segment (start 98.76502 94.33498) (end 97.63 95.47) (width 0.25) (layer F.Cu) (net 28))
 (segment (start 100.9708 94.33498) (end 98.76502 94.33498) (width 0.25) (layer F.Cu) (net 28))
 (segment (start 97.63 99.92) (end 97.59 99.96) (width 0.25) (layer B.Cu) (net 28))
 (segment (start 97.63 95.47) (end 97.63 99.92) (width 0.25) (layer B.Cu) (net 28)))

